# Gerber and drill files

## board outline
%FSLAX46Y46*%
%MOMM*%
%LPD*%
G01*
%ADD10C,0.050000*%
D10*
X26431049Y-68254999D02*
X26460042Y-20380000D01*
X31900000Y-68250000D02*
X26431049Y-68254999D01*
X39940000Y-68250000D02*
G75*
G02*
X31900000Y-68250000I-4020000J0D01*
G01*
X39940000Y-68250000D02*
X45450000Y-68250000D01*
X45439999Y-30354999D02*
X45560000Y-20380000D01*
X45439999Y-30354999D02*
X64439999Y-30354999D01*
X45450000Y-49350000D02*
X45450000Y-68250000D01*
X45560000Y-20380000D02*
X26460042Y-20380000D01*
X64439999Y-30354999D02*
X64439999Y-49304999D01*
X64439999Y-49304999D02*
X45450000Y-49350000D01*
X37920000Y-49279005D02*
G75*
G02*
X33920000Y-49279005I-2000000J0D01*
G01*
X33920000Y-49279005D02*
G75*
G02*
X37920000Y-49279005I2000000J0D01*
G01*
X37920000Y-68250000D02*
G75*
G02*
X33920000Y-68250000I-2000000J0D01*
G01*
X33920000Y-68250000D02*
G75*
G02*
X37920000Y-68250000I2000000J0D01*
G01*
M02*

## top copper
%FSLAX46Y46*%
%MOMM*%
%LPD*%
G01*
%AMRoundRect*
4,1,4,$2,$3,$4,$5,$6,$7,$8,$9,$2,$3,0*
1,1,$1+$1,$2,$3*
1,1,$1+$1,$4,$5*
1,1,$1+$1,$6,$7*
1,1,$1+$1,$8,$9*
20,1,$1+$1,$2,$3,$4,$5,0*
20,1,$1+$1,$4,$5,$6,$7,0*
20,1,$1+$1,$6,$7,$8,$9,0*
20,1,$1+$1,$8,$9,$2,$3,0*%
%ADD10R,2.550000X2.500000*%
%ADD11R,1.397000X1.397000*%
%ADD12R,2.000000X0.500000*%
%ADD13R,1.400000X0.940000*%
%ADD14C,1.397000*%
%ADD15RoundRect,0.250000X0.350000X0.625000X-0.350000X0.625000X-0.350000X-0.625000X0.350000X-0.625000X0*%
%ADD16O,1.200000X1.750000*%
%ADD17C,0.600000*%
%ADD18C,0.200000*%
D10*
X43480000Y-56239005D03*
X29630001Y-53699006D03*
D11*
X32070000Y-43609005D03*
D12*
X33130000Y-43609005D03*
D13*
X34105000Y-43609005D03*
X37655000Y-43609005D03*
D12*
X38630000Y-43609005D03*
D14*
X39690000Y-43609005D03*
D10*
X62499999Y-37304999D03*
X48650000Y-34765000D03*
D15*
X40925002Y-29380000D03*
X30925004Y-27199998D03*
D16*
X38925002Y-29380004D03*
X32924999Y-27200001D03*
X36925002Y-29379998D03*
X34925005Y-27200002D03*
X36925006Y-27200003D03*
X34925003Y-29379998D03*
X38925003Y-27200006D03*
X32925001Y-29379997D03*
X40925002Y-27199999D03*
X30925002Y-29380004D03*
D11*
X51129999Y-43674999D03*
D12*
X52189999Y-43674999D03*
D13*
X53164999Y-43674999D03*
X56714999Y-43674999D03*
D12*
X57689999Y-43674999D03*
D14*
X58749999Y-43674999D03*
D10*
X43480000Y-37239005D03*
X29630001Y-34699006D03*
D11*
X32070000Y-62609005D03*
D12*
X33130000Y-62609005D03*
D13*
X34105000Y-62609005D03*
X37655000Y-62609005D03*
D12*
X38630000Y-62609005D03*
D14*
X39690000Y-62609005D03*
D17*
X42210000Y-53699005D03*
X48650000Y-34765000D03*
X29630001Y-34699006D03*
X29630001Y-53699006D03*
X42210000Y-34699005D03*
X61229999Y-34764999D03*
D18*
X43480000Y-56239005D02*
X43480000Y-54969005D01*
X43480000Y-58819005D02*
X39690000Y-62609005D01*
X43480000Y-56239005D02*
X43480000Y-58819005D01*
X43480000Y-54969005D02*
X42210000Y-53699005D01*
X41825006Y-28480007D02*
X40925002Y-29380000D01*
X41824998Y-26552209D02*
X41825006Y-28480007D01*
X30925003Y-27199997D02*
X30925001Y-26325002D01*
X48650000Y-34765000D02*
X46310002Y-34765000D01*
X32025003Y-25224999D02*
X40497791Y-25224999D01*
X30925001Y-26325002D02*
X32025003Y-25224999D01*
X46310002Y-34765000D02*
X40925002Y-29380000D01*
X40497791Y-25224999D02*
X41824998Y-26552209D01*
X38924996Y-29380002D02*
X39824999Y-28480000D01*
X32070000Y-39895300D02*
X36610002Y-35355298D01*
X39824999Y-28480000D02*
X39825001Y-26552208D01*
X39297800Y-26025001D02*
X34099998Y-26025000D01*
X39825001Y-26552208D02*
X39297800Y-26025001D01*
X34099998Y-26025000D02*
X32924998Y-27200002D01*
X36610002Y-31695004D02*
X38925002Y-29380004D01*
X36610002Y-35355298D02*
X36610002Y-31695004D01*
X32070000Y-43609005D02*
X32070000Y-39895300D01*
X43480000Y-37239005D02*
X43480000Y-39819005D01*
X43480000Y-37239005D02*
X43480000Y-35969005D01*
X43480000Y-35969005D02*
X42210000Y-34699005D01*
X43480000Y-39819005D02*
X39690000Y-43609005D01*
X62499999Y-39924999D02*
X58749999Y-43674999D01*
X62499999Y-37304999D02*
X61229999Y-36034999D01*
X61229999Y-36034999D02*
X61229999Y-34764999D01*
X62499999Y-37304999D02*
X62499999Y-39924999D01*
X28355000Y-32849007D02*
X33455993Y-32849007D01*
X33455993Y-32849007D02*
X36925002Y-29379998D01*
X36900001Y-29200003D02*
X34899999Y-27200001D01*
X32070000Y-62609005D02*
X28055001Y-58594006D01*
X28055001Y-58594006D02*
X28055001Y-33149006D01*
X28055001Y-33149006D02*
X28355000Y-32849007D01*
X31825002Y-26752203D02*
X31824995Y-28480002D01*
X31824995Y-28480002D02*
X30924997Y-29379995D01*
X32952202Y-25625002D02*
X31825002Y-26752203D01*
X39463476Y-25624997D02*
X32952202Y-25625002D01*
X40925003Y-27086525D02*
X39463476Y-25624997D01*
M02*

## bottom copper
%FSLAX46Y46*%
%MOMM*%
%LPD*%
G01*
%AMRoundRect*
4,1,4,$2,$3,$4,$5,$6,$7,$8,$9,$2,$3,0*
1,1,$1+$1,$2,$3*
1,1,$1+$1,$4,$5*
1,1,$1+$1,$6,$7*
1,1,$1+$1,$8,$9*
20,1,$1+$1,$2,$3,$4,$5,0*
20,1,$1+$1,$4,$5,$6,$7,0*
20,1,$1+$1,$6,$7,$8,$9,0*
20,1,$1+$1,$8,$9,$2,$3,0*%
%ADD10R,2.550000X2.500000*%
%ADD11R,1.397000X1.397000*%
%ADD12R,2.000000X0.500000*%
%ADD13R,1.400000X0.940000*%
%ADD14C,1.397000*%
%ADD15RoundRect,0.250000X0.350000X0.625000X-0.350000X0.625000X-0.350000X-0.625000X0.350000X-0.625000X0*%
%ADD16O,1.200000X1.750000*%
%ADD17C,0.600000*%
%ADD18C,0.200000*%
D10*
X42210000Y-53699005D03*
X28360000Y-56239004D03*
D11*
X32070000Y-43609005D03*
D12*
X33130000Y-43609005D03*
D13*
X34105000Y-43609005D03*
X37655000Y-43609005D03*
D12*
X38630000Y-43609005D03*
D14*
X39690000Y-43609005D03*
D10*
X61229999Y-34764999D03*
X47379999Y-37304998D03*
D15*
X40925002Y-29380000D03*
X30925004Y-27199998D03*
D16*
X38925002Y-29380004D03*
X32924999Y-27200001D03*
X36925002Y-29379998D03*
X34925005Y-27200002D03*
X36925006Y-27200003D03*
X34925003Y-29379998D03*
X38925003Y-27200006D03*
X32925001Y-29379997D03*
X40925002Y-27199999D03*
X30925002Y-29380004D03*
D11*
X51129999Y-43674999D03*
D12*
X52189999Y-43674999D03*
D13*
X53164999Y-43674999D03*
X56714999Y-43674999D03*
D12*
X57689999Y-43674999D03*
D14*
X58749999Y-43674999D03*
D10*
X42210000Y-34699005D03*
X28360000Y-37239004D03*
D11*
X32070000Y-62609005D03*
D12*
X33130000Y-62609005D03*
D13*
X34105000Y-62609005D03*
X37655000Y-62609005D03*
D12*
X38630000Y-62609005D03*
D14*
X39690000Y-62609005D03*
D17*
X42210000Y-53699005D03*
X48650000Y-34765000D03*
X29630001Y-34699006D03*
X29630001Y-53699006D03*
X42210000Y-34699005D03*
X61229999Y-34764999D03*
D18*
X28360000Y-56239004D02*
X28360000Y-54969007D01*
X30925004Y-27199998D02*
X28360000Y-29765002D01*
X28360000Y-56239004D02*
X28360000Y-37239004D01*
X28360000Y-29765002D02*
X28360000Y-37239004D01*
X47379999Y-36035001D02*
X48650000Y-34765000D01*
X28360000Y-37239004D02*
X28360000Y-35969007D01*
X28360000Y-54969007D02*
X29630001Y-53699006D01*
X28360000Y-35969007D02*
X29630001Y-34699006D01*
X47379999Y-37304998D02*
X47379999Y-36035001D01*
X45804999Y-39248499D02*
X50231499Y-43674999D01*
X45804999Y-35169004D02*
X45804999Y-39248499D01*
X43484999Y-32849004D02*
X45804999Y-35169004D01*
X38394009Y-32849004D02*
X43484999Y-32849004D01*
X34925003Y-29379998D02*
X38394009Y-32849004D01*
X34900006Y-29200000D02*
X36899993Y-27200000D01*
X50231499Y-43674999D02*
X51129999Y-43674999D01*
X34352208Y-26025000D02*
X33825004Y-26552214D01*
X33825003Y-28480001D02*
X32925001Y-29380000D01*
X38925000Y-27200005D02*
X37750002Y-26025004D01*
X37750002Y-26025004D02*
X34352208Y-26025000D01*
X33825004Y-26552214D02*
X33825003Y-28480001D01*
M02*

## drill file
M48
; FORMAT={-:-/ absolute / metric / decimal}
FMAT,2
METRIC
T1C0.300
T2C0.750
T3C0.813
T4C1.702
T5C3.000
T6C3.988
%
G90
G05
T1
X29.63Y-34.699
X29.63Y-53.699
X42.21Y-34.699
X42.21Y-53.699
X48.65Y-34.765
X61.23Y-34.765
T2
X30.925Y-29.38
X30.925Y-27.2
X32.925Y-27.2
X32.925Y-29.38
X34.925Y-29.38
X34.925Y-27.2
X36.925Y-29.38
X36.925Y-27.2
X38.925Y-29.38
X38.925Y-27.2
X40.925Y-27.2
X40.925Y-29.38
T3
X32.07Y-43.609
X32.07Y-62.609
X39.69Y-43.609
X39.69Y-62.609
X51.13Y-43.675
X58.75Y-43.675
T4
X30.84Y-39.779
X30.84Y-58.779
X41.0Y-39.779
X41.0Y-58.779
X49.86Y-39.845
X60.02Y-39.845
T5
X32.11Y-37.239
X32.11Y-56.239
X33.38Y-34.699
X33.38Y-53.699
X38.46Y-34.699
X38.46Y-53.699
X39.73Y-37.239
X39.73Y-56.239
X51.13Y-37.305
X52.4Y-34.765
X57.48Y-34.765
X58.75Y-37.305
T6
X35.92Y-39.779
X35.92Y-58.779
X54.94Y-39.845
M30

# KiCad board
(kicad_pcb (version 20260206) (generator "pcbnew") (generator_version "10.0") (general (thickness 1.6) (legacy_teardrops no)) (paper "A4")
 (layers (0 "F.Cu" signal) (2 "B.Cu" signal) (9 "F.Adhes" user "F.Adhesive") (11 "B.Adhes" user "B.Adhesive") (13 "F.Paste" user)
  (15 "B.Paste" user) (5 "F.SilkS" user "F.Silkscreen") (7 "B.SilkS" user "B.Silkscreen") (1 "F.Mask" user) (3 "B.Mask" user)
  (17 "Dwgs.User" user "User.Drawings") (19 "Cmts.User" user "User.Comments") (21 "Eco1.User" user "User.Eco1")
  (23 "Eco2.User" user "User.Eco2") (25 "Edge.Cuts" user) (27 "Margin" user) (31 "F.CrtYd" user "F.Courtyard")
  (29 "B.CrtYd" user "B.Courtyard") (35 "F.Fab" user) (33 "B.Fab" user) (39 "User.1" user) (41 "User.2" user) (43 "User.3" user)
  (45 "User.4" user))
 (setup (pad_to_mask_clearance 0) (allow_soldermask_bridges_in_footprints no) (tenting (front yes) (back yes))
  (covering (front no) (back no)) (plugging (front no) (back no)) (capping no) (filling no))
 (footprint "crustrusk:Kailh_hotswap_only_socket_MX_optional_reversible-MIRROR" (layer "F.Cu") (at 35.92 58.779005)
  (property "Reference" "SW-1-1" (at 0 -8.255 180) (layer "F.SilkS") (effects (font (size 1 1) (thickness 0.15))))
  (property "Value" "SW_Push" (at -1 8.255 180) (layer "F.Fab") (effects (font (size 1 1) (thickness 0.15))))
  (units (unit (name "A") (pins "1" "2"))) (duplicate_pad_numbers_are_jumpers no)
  (pad "" np_thru_hole circle (at -5.08 0) (size 1.7018 1.7018) (drill 1.7018) (layers "*.Cu" "*.Mask"))
  (pad "" np_thru_hole circle (at -3.81 -2.54 180) (size 3 3) (drill 3) (layers "*.Cu" "*.Mask"))
  (pad "" np_thru_hole circle (at -2.54 -5.079998) (size 3 3) (drill 3) (layers "*.Cu" "*.Mask"))
  (pad "" np_thru_hole circle (at 0 0) (size 3.9878 3.9878) (drill 3.9878) (layers "*.Cu" "*.Mask"))
  (pad "" np_thru_hole circle (at 2.540002 -5.080001 180) (size 3 3) (drill 3) (layers "*.Cu" "*.Mask"))
  (pad "" np_thru_hole circle (at 3.81 -2.54) (size 3 3) (drill 3) (layers "*.Cu" "*.Mask"))
  (pad "" np_thru_hole circle (at 5.08 0) (size 1.7018 1.7018) (drill 1.7018) (layers "*.Cu" "*.Mask"))
  (pad "1" smd rect (at 6.29 -5.08 180) (size 2.55 2.5) (layers "B.Cu" "B.Mask" "B.Paste") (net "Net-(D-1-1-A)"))
  (pad "1" smd rect (at 7.56 -2.54) (size 2.55 2.5) (layers "F.Cu" "F.Mask" "F.Paste") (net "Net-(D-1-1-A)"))
  (pad "2" smd rect (at -7.56 -2.540001 180) (size 2.55 2.5) (layers "B.Cu" "B.Mask" "B.Paste") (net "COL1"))
  (pad "2" smd rect (at -6.289999 -5.079999) (size 2.55 2.5) (layers "F.Cu" "F.Mask" "F.Paste") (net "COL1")))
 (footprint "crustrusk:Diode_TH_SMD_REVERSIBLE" (layer "F.Cu") (at 35.88 43.609005)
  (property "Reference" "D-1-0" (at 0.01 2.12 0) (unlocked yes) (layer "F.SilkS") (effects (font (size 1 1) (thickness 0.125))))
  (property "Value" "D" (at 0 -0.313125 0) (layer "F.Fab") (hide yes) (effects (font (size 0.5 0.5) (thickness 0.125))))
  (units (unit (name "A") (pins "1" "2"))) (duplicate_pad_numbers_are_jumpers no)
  (pad "1" thru_hole rect (at -3.81 0) (size 1.397 1.397) (drill 0.8128) (layers "*.Cu" "*.Mask") (remove_unused_layers no) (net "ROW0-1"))
  (pad "1" smd rect (at -2.75 0 180) (size 2 0.5) (layers "F.Cu") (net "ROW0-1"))
  (pad "1" smd rect (at -2.75 0) (size 2 0.5) (layers "B.Cu") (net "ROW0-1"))
  (pad "1" smd rect (at -1.775 0 180) (size 1.4 0.94) (layers "F.Cu" "F.Mask" "F.Paste") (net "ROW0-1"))
  (pad "1" smd rect (at -1.775 0) (size 1.4 0.94) (layers "B.Cu" "B.Mask" "B.Paste") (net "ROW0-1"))
  (pad "2" smd rect (at 1.775 0 180) (size 1.4 0.94) (layers "F.Cu" "F.Mask" "F.Paste") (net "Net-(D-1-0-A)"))
  (pad "2" smd rect (at 1.775 0) (size 1.4 0.94) (layers "B.Cu" "B.Mask" "B.Paste") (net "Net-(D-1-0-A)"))
  (pad "2" smd rect (at 2.75 0 180) (size 2 0.5) (layers "F.Cu") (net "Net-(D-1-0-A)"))
  (pad "2" smd rect (at 2.75 0) (size 2 0.5) (layers "B.Cu") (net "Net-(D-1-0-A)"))
  (pad "2" thru_hole circle (at 3.81 0) (size 1.397 1.397) (drill 0.8128) (layers "*.Cu" "*.Mask") (remove_unused_layers no)
   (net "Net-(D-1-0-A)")))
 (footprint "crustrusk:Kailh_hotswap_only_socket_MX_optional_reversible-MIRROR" (layer "F.Cu") (at 54.939999 39.844999)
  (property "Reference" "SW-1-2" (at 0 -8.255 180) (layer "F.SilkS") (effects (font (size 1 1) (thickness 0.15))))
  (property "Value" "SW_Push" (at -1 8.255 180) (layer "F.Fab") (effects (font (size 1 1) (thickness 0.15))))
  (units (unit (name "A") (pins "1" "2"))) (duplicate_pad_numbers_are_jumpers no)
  (pad "" np_thru_hole circle (at -5.08 0) (size 1.7018 1.7018) (drill 1.7018) (layers "*.Cu" "*.Mask"))
  (pad "" np_thru_hole circle (at -3.81 -2.54 180) (size 3 3) (drill 3) (layers "*.Cu" "*.Mask"))
  (pad "" np_thru_hole circle (at -2.54 -5.079998) (size 3 3) (drill 3) (layers "*.Cu" "*.Mask"))
  (pad "" np_thru_hole circle (at 0 0) (size 3.9878 3.9878) (drill 3.9878) (layers "*.Cu" "*.Mask"))
  (pad "" np_thru_hole circle (at 2.540002 -5.080001 180) (size 3 3) (drill 3) (layers "*.Cu" "*.Mask"))
  (pad "" np_thru_hole circle (at 3.81 -2.54) (size 3 3) (drill 3) (layers "*.Cu" "*.Mask"))
  (pad "" np_thru_hole circle (at 5.08 0) (size 1.7018 1.7018) (drill 1.7018) (layers "*.Cu" "*.Mask"))
  (pad "1" smd rect (at 6.29 -5.08 180) (size 2.55 2.5) (layers "B.Cu" "B.Mask" "B.Paste") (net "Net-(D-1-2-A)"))
  (pad "1" smd rect (at 7.56 -2.54) (size 2.55 2.5) (layers "F.Cu" "F.Mask" "F.Paste") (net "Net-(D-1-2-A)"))
  (pad "2" smd rect (at -7.56 -2.540001 180) (size 2.55 2.5) (layers "B.Cu" "B.Mask" "B.Paste") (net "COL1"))
  (pad "2" smd rect (at -6.289999 -5.079999) (size 2.55 2.5) (layers "F.Cu" "F.Mask" "F.Paste") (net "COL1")))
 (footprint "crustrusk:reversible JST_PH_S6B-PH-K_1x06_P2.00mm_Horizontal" (layer "F.Cu") (at 40.925002 29.38 180)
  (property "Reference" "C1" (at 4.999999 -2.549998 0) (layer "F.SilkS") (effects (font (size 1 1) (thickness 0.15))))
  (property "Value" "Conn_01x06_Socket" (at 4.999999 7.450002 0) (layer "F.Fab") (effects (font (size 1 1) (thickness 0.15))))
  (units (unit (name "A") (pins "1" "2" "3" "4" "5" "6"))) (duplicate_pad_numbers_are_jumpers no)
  (pad "1" thru_hole roundrect (at 0 0 180) (size 1.2 1.75) (drill 0.75) (layers "*.Cu" "*.Mask") (remove_unused_layers no)
   (roundrect_rratio 0.208333) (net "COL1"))
  (pad "1" thru_hole roundrect (at 9.999998 2.180002 180) (size 1.2 1.75) (drill 0.75) (layers "*.Cu" "*.Mask") (remove_unused_layers no)
   (roundrect_rratio 0.208333) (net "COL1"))
  (pad "2" thru_hole oval (at 2 -0.000004 180) (size 1.2 1.75) (drill 0.75) (layers "*.Cu" "*.Mask") (remove_unused_layers no)
   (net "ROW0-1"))
  (pad "2" thru_hole oval (at 8.000003 2.179999 180) (size 1.2 1.75) (drill 0.75) (layers "*.Cu" "*.Mask") (remove_unused_layers no)
   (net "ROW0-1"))
  (pad "3" thru_hole oval (at 4 0.000002 180) (size 1.2 1.75) (drill 0.75) (layers "*.Cu" "*.Mask") (remove_unused_layers no) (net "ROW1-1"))
  (pad "3" thru_hole oval (at 5.999997 2.179998 180) (size 1.2 1.75) (drill 0.75) (layers "*.Cu" "*.Mask") (remove_unused_layers no)
   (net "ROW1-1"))
  (pad "4" thru_hole oval (at 3.999996 2.179997 180) (size 1.2 1.75) (drill 0.75) (layers "*.Cu" "*.Mask") (remove_unused_layers no)
   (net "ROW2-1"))
  (pad "4" thru_hole oval (at 5.999999 0.000002 180) (size 1.2 1.75) (drill 0.75) (layers "*.Cu" "*.Mask") (remove_unused_layers no)
   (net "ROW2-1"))
  (pad "5" thru_hole oval (at 1.999999 2.179994 180) (size 1.2 1.75) (drill 0.75) (layers "*.Cu" "*.Mask") (remove_unused_layers no)
   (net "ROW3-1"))
  (pad "5" thru_hole oval (at 8.000001 0.000003 180) (size 1.2 1.75) (drill 0.75) (layers "*.Cu" "*.Mask") (remove_unused_layers no)
   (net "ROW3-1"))
  (pad "6" thru_hole oval (at 0 2.180001 180) (size 1.2 1.75) (drill 0.75) (layers "*.Cu" "*.Mask") (remove_unused_layers no) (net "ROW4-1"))
  (pad "6" thru_hole oval (at 10 -0.000004 180) (size 1.2 1.75) (drill 0.75) (layers "*.Cu" "*.Mask") (remove_unused_layers no)
   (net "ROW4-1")))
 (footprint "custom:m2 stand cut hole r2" (layer "F.Cu") (at 35.92 49.279005)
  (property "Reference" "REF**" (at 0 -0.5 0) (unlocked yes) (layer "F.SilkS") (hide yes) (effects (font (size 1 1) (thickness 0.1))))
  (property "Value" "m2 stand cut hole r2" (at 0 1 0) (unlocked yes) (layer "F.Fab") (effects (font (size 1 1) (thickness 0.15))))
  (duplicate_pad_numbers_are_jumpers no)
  (fp_circle (center 0 0) (end 2 0) (stroke (width 0.05) (type default)) (fill no) (layer "Edge.Cuts")))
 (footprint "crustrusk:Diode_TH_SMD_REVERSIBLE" (layer "F.Cu") (at 54.939999 43.674999)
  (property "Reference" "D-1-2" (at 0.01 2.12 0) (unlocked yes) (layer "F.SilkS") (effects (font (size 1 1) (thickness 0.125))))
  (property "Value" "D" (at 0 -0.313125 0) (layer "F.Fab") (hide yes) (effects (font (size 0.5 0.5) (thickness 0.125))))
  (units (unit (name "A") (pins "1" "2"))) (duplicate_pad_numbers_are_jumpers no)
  (pad "1" thru_hole rect (at -3.81 0) (size 1.397 1.397) (drill 0.8128) (layers "*.Cu" "*.Mask") (remove_unused_layers no) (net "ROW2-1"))
  (pad "1" smd rect (at -2.75 0 180) (size 2 0.5) (layers "F.Cu") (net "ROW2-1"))
  (pad "1" smd rect (at -2.75 0) (size 2 0.5) (layers "B.Cu") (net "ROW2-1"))
  (pad "1" smd rect (at -1.775 0 180) (size 1.4 0.94) (layers "F.Cu" "F.Mask" "F.Paste") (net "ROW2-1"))
  (pad "1" smd rect (at -1.775 0) (size 1.4 0.94) (layers "B.Cu" "B.Mask" "B.Paste") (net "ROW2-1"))
  (pad "2" smd rect (at 1.775 0 180) (size 1.4 0.94) (layers "F.Cu" "F.Mask" "F.Paste") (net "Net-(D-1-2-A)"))
  (pad "2" smd rect (at 1.775 0) (size 1.4 0.94) (layers "B.Cu" "B.Mask" "B.Paste") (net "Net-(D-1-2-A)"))
  (pad "2" smd rect (at 2.75 0 180) (size 2 0.5) (layers "F.Cu") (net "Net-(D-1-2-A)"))
  (pad "2" smd rect (at 2.75 0) (size 2 0.5) (layers "B.Cu") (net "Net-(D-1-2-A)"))
  (pad "2" thru_hole circle (at 3.81 0) (size 1.397 1.397) (drill 0.8128) (layers "*.Cu" "*.Mask") (remove_unused_layers no)
   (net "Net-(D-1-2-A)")))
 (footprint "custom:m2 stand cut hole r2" (layer "F.Cu") (at 35.92 68.25)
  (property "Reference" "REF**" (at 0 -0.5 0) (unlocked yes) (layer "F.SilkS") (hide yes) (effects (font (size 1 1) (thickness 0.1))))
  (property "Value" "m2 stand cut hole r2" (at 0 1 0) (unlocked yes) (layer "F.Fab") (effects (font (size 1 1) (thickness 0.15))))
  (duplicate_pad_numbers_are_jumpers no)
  (fp_circle (center 0 0) (end 2 0) (stroke (width 0.05) (type default)) (fill no) (layer "Edge.Cuts")))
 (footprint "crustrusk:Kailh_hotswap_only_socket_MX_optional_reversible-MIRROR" (layer "F.Cu") (at 35.92 39.779005)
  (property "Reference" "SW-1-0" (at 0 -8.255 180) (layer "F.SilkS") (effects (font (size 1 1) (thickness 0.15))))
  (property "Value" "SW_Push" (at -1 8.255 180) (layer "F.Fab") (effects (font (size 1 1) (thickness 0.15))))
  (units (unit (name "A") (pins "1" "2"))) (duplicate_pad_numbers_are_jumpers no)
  (pad "" np_thru_hole circle (at -5.08 0) (size 1.7018 1.7018) (drill 1.7018) (layers "*.Cu" "*.Mask"))
  (pad "" np_thru_hole circle (at -3.81 -2.54 180) (size 3 3) (drill 3) (layers "*.Cu" "*.Mask"))
  (pad "" np_thru_hole circle (at -2.54 -5.079998) (size 3 3) (drill 3) (layers "*.Cu" "*.Mask"))
  (pad "" np_thru_hole circle (at 0 0) (size 3.9878 3.9878) (drill 3.9878) (layers "*.Cu" "*.Mask"))
  (pad "" np_thru_hole circle (at 2.540002 -5.080001 180) (size 3 3) (drill 3) (layers "*.Cu" "*.Mask"))
  (pad "" np_thru_hole circle (at 3.81 -2.54) (size 3 3) (drill 3) (layers "*.Cu" "*.Mask"))
  (pad "" np_thru_hole circle (at 5.08 0) (size 1.7018 1.7018) (drill 1.7018) (layers "*.Cu" "*.Mask"))
  (pad "1" smd rect (at 6.29 -5.08 180) (size 2.55 2.5) (layers "B.Cu" "B.Mask" "B.Paste") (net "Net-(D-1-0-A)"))
  (pad "1" smd rect (at 7.56 -2.54) (size 2.55 2.5) (layers "F.Cu" "F.Mask" "F.Paste") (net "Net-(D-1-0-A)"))
  (pad "2" smd rect (at -7.56 -2.540001 180) (size 2.55 2.5) (layers "B.Cu" "B.Mask" "B.Paste") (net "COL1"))
  (pad "2" smd rect (at -6.289999 -5.079999) (size 2.55 2.5) (layers "F.Cu" "F.Mask" "F.Paste") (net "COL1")))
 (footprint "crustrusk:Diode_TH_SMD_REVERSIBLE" (layer "F.Cu") (at 35.88 62.609005)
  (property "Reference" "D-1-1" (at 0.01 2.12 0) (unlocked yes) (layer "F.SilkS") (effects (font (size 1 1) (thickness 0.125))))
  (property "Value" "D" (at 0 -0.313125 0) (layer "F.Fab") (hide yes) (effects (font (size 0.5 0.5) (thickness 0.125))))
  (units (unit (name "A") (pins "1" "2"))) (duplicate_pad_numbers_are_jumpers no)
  (pad "1" thru_hole rect (at -3.81 0) (size 1.397 1.397) (drill 0.8128) (layers "*.Cu" "*.Mask") (remove_unused_layers no) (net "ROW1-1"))
  (pad "1" smd rect (at -2.75 0 180) (size 2 0.5) (layers "F.Cu") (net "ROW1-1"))
  (pad "1" smd rect (at -2.75 0) (size 2 0.5) (layers "B.Cu") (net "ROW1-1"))
  (pad "1" smd rect (at -1.775 0 180) (size 1.4 0.94) (layers "F.Cu" "F.Mask" "F.Paste") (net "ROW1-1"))
  (pad "1" smd rect (at -1.775 0) (size 1.4 0.94) (layers "B.Cu" "B.Mask" "B.Paste") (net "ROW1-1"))
  (pad "2" smd rect (at 1.775 0 180) (size 1.4 0.94) (layers "F.Cu" "F.Mask" "F.Paste") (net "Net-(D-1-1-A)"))
  (pad "2" smd rect (at 1.775 0) (size 1.4 0.94) (layers "B.Cu" "B.Mask" "B.Paste") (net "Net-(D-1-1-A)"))
  (pad "2" smd rect (at 2.75 0 180) (size 2 0.5) (layers "F.Cu") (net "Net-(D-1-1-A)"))
  (pad "2" smd rect (at 2.75 0) (size 2 0.5) (layers "B.Cu") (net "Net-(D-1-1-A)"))
  (pad "2" thru_hole circle (at 3.81 0) (size 1.397 1.397) (drill 0.8128) (layers "*.Cu" "*.Mask") (remove_unused_layers no)
   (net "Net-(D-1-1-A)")))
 (gr_line (start 26.431049 68.254999) (end 26.460042 20.38) (stroke (width 0.05) (type default)) (layer "Edge.Cuts"))
 (gr_line (start 31.9 68.25) (end 26.431049 68.254999) (stroke (width 0.05) (type default)) (layer "Edge.Cuts"))
 (gr_arc (start 39.94 68.25) (mid 35.92 72.27) (end 31.9 68.25) (stroke (width 0.05) (type default)) (layer "Edge.Cuts"))
 (gr_line (start 39.94 68.25) (end 45.45 68.25) (stroke (width 0.05) (type default)) (layer "Edge.Cuts"))
 (gr_line (start 45.439999 30.354999) (end 45.56 20.38) (stroke (width 0.05) (type default)) (layer "Edge.Cuts"))
 (gr_line (start 45.439999 30.354999) (end 64.439999 30.354999) (stroke (width 0.05) (type default)) (layer "Edge.Cuts"))
 (gr_line (start 45.45 49.35) (end 45.45 68.25) (stroke (width 0.05) (type default)) (layer "Edge.Cuts"))
 (gr_line (start 45.56 20.38) (end 26.460042 20.38) (stroke (width 0.05) (type default)) (layer "Edge.Cuts"))
 (gr_line (start 64.439999 30.354999) (end 64.439999 49.304999) (stroke (width 0.05) (type default)) (layer "Edge.Cuts"))
 (gr_line (start 64.439999 49.304999) (end 45.45 49.35) (stroke (width 0.05) (type default)) (layer "Edge.Cuts"))
 (segment (start 43.48 56.239005) (end 43.48 54.969005) (width 0.2) (layer "F.Cu") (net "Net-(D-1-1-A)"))
 (segment (start 43.48 58.819005) (end 39.69 62.609005) (width 0.2) (layer "F.Cu") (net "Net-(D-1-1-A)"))
 (segment (start 43.48 56.239005) (end 43.48 58.819005) (width 0.2) (layer "F.Cu") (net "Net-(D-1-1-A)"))
 (segment (start 43.48 54.969005) (end 42.21 53.699005) (width 0.2) (layer "F.Cu") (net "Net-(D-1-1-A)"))
 (via (at 42.21 53.699005) (size 0.6) (drill 0.3) (layers "F.Cu" "B.Cu") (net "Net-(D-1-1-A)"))
 (segment (start 41.825006 28.480007) (end 40.925002 29.38) (width 0.2) (layer "F.Cu") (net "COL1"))
 (segment (start 41.824998 26.552209) (end 41.825006 28.480007) (width 0.2) (layer "F.Cu") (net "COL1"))
 (segment (start 30.925003 27.199997) (end 30.925001 26.325002) (width 0.2) (layer "F.Cu") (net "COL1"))
 (segment (start 48.65 34.765) (end 46.310002 34.765) (width 0.2) (layer "F.Cu") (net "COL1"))
 (segment (start 32.025003 25.224999) (end 40.497791 25.224999) (width 0.2) (layer "F.Cu") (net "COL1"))
 (segment (start 30.925001 26.325002) (end 32.025003 25.224999) (width 0.2) (layer "F.Cu") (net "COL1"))
 (segment (start 46.310002 34.765) (end 40.925002 29.38) (width 0.2) (layer "F.Cu") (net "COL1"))
 (segment (start 40.497791 25.224999) (end 41.824998 26.552209) (width 0.2) (layer "F.Cu") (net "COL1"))
 (via (at 48.65 34.765) (size 0.6) (drill 0.3) (layers "F.Cu" "B.Cu") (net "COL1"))
 (via (at 29.630001 34.699006) (size 0.6) (drill 0.3) (layers "F.Cu" "B.Cu") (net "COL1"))
 (via (at 29.630001 53.699006) (size 0.6) (drill 0.3) (layers "F.Cu" "B.Cu") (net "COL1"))
 (segment (start 28.36 56.239004) (end 28.36 54.969007) (width 0.2) (layer "B.Cu") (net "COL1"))
 (segment (start 30.925004 27.199998) (end 28.36 29.765002) (width 0.2) (layer "B.Cu") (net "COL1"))
 (segment (start 28.36 56.239004) (end 28.36 37.239004) (width 0.2) (layer "B.Cu") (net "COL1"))
 (segment (start 28.36 29.765002) (end 28.36 37.239004) (width 0.2) (layer "B.Cu") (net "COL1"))
 (segment (start 47.379999 36.035001) (end 48.65 34.765) (width 0.2) (layer "B.Cu") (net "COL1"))
 (segment (start 28.36 37.239004) (end 28.36 35.969007) (width 0.2) (layer "B.Cu") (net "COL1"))
 (segment (start 28.36 54.969007) (end 29.630001 53.699006) (width 0.2) (layer "B.Cu") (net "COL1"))
 (segment (start 28.36 35.969007) (end 29.630001 34.699006) (width 0.2) (layer "B.Cu") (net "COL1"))
 (segment (start 47.379999 37.304998) (end 47.379999 36.035001) (width 0.2) (layer "B.Cu") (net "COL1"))
 (segment (start 38.924996 29.380002) (end 39.824999 28.48) (width 0.2) (layer "F.Cu") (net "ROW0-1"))
 (segment (start 32.07 39.8953) (end 36.610002 35.355298) (width 0.2) (layer "F.Cu") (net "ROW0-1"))
 (segment (start 39.824999 28.48) (end 39.825001 26.552208) (width 0.2) (layer "F.Cu") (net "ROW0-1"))
 (segment (start 39.2978 26.025001) (end 34.099998 26.025) (width 0.2) (layer "F.Cu") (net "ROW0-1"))
 (segment (start 39.825001 26.552208) (end 39.2978 26.025001) (width 0.2) (layer "F.Cu") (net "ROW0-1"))
 (segment (start 34.099998 26.025) (end 32.924998 27.200002) (width 0.2) (layer "F.Cu") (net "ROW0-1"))
 (segment (start 36.610002 31.695004) (end 38.925002 29.380004) (width 0.2) (layer "F.Cu") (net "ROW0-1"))
 (segment (start 36.610002 35.355298) (end 36.610002 31.695004) (width 0.2) (layer "F.Cu") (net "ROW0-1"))
 (segment (start 32.07 43.609005) (end 32.07 39.8953) (width 0.2) (layer "F.Cu") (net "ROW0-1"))
 (segment (start 43.48 37.239005) (end 43.48 39.819005) (width 0.2) (layer "F.Cu") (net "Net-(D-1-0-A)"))
 (segment (start 43.48 37.239005) (end 43.48 35.969005) (width 0.2) (layer "F.Cu") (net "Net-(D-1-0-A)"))
 (segment (start 43.48 35.969005) (end 42.21 34.699005) (width 0.2) (layer "F.Cu") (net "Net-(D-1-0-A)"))
 (segment (start 43.48 39.819005) (end 39.69 43.609005) (width 0.2) (layer "F.Cu") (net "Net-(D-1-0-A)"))
 (via (at 42.21 34.699005) (size 0.6) (drill 0.3) (layers "F.Cu" "B.Cu") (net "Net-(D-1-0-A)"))
 (segment (start 62.499999 39.924999) (end 58.749999 43.674999) (width 0.2) (layer "F.Cu") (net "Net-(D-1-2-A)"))
 (segment (start 62.499999 37.304999) (end 61.229999 36.034999) (width 0.2) (layer "F.Cu") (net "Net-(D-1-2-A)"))
 (segment (start 61.229999 36.034999) (end 61.229999 34.764999) (width 0.2) (layer "F.Cu") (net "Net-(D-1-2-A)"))
 (segment (start 62.499999 37.304999) (end 62.499999 39.924999) (width 0.2) (layer "F.Cu") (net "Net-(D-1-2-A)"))
 (via (at 61.229999 34.764999) (size 0.6) (drill 0.3) (layers "F.Cu" "B.Cu") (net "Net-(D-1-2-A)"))
 (segment (start 28.355 32.849007) (end 33.455993 32.849007) (width 0.2) (layer "F.Cu") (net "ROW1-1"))
 (segment (start 33.455993 32.849007) (end 36.925002 29.379998) (width 0.2) (layer "F.Cu") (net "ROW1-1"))
 (segment (start 36.900001 29.200003) (end 34.899999 27.200001) (width 0.2) (layer "F.Cu") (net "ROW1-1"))
 (segment (start 32.07 62.609005) (end 28.055001 58.594006) (width 0.2) (layer "F.Cu") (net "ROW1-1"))
 (segment (start 28.055001 58.594006) (end 28.055001 33.149006) (width 0.2) (layer "F.Cu") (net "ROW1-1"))
 (segment (start 28.055001 33.149006) (end 28.355 32.849007) (width 0.2) (layer "F.Cu") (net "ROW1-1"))
 (segment (start 45.804999 39.248499) (end 50.231499 43.674999) (width 0.2) (layer "B.Cu") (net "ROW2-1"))
 (segment (start 45.804999 35.169004) (end 45.804999 39.248499) (width 0.2) (layer "B.Cu") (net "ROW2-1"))
 (segment (start 43.484999 32.849004) (end 45.804999 35.169004) (width 0.2) (layer "B.Cu") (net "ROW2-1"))
 (segment (start 38.394009 32.849004) (end 43.484999 32.849004) (width 0.2) (layer "B.Cu") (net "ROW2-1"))
 (segment (start 34.925003 29.379998) (end 38.394009 32.849004) (width 0.2) (layer "B.Cu") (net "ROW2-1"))
 (segment (start 34.900006 29.2) (end 36.899993 27.2) (width 0.2) (layer "B.Cu") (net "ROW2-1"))
 (segment (start 50.231499 43.674999) (end 51.129999 43.674999) (width 0.2) (layer "B.Cu") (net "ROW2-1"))
 (segment (start 34.352208 26.025) (end 33.825004 26.552214) (width 0.2) (layer "B.Cu") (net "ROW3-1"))
 (segment (start 33.825003 28.480001) (end 32.925001 29.38) (width 0.2) (layer "B.Cu") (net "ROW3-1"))
 (segment (start 38.925 27.200005) (end 37.750002 26.025004) (width 0.2) (layer "B.Cu") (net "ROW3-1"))
 (segment (start 37.750002 26.025004) (end 34.352208 26.025) (width 0.2) (layer "B.Cu") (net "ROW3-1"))
 (segment (start 33.825004 26.552214) (end 33.825003 28.480001) (width 0.2) (layer "B.Cu") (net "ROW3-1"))
 (segment (start 31.825002 26.752203) (end 31.824995 28.480002) (width 0.2) (layer "F.Cu") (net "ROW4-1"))
 (segment (start 31.824995 28.480002) (end 30.924997 29.379995) (width 0.2) (layer "F.Cu") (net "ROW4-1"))
 (segment (start 32.952202 25.625002) (end 31.825002 26.752203) (width 0.2) (layer "F.Cu") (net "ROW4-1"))
 (segment (start 39.463476 25.624997) (end 32.952202 25.625002) (width 0.2) (layer "F.Cu") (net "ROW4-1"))
 (segment (start 40.925003 27.086525) (end 39.463476 25.624997) (width 0.2) (layer "F.Cu") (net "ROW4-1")))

